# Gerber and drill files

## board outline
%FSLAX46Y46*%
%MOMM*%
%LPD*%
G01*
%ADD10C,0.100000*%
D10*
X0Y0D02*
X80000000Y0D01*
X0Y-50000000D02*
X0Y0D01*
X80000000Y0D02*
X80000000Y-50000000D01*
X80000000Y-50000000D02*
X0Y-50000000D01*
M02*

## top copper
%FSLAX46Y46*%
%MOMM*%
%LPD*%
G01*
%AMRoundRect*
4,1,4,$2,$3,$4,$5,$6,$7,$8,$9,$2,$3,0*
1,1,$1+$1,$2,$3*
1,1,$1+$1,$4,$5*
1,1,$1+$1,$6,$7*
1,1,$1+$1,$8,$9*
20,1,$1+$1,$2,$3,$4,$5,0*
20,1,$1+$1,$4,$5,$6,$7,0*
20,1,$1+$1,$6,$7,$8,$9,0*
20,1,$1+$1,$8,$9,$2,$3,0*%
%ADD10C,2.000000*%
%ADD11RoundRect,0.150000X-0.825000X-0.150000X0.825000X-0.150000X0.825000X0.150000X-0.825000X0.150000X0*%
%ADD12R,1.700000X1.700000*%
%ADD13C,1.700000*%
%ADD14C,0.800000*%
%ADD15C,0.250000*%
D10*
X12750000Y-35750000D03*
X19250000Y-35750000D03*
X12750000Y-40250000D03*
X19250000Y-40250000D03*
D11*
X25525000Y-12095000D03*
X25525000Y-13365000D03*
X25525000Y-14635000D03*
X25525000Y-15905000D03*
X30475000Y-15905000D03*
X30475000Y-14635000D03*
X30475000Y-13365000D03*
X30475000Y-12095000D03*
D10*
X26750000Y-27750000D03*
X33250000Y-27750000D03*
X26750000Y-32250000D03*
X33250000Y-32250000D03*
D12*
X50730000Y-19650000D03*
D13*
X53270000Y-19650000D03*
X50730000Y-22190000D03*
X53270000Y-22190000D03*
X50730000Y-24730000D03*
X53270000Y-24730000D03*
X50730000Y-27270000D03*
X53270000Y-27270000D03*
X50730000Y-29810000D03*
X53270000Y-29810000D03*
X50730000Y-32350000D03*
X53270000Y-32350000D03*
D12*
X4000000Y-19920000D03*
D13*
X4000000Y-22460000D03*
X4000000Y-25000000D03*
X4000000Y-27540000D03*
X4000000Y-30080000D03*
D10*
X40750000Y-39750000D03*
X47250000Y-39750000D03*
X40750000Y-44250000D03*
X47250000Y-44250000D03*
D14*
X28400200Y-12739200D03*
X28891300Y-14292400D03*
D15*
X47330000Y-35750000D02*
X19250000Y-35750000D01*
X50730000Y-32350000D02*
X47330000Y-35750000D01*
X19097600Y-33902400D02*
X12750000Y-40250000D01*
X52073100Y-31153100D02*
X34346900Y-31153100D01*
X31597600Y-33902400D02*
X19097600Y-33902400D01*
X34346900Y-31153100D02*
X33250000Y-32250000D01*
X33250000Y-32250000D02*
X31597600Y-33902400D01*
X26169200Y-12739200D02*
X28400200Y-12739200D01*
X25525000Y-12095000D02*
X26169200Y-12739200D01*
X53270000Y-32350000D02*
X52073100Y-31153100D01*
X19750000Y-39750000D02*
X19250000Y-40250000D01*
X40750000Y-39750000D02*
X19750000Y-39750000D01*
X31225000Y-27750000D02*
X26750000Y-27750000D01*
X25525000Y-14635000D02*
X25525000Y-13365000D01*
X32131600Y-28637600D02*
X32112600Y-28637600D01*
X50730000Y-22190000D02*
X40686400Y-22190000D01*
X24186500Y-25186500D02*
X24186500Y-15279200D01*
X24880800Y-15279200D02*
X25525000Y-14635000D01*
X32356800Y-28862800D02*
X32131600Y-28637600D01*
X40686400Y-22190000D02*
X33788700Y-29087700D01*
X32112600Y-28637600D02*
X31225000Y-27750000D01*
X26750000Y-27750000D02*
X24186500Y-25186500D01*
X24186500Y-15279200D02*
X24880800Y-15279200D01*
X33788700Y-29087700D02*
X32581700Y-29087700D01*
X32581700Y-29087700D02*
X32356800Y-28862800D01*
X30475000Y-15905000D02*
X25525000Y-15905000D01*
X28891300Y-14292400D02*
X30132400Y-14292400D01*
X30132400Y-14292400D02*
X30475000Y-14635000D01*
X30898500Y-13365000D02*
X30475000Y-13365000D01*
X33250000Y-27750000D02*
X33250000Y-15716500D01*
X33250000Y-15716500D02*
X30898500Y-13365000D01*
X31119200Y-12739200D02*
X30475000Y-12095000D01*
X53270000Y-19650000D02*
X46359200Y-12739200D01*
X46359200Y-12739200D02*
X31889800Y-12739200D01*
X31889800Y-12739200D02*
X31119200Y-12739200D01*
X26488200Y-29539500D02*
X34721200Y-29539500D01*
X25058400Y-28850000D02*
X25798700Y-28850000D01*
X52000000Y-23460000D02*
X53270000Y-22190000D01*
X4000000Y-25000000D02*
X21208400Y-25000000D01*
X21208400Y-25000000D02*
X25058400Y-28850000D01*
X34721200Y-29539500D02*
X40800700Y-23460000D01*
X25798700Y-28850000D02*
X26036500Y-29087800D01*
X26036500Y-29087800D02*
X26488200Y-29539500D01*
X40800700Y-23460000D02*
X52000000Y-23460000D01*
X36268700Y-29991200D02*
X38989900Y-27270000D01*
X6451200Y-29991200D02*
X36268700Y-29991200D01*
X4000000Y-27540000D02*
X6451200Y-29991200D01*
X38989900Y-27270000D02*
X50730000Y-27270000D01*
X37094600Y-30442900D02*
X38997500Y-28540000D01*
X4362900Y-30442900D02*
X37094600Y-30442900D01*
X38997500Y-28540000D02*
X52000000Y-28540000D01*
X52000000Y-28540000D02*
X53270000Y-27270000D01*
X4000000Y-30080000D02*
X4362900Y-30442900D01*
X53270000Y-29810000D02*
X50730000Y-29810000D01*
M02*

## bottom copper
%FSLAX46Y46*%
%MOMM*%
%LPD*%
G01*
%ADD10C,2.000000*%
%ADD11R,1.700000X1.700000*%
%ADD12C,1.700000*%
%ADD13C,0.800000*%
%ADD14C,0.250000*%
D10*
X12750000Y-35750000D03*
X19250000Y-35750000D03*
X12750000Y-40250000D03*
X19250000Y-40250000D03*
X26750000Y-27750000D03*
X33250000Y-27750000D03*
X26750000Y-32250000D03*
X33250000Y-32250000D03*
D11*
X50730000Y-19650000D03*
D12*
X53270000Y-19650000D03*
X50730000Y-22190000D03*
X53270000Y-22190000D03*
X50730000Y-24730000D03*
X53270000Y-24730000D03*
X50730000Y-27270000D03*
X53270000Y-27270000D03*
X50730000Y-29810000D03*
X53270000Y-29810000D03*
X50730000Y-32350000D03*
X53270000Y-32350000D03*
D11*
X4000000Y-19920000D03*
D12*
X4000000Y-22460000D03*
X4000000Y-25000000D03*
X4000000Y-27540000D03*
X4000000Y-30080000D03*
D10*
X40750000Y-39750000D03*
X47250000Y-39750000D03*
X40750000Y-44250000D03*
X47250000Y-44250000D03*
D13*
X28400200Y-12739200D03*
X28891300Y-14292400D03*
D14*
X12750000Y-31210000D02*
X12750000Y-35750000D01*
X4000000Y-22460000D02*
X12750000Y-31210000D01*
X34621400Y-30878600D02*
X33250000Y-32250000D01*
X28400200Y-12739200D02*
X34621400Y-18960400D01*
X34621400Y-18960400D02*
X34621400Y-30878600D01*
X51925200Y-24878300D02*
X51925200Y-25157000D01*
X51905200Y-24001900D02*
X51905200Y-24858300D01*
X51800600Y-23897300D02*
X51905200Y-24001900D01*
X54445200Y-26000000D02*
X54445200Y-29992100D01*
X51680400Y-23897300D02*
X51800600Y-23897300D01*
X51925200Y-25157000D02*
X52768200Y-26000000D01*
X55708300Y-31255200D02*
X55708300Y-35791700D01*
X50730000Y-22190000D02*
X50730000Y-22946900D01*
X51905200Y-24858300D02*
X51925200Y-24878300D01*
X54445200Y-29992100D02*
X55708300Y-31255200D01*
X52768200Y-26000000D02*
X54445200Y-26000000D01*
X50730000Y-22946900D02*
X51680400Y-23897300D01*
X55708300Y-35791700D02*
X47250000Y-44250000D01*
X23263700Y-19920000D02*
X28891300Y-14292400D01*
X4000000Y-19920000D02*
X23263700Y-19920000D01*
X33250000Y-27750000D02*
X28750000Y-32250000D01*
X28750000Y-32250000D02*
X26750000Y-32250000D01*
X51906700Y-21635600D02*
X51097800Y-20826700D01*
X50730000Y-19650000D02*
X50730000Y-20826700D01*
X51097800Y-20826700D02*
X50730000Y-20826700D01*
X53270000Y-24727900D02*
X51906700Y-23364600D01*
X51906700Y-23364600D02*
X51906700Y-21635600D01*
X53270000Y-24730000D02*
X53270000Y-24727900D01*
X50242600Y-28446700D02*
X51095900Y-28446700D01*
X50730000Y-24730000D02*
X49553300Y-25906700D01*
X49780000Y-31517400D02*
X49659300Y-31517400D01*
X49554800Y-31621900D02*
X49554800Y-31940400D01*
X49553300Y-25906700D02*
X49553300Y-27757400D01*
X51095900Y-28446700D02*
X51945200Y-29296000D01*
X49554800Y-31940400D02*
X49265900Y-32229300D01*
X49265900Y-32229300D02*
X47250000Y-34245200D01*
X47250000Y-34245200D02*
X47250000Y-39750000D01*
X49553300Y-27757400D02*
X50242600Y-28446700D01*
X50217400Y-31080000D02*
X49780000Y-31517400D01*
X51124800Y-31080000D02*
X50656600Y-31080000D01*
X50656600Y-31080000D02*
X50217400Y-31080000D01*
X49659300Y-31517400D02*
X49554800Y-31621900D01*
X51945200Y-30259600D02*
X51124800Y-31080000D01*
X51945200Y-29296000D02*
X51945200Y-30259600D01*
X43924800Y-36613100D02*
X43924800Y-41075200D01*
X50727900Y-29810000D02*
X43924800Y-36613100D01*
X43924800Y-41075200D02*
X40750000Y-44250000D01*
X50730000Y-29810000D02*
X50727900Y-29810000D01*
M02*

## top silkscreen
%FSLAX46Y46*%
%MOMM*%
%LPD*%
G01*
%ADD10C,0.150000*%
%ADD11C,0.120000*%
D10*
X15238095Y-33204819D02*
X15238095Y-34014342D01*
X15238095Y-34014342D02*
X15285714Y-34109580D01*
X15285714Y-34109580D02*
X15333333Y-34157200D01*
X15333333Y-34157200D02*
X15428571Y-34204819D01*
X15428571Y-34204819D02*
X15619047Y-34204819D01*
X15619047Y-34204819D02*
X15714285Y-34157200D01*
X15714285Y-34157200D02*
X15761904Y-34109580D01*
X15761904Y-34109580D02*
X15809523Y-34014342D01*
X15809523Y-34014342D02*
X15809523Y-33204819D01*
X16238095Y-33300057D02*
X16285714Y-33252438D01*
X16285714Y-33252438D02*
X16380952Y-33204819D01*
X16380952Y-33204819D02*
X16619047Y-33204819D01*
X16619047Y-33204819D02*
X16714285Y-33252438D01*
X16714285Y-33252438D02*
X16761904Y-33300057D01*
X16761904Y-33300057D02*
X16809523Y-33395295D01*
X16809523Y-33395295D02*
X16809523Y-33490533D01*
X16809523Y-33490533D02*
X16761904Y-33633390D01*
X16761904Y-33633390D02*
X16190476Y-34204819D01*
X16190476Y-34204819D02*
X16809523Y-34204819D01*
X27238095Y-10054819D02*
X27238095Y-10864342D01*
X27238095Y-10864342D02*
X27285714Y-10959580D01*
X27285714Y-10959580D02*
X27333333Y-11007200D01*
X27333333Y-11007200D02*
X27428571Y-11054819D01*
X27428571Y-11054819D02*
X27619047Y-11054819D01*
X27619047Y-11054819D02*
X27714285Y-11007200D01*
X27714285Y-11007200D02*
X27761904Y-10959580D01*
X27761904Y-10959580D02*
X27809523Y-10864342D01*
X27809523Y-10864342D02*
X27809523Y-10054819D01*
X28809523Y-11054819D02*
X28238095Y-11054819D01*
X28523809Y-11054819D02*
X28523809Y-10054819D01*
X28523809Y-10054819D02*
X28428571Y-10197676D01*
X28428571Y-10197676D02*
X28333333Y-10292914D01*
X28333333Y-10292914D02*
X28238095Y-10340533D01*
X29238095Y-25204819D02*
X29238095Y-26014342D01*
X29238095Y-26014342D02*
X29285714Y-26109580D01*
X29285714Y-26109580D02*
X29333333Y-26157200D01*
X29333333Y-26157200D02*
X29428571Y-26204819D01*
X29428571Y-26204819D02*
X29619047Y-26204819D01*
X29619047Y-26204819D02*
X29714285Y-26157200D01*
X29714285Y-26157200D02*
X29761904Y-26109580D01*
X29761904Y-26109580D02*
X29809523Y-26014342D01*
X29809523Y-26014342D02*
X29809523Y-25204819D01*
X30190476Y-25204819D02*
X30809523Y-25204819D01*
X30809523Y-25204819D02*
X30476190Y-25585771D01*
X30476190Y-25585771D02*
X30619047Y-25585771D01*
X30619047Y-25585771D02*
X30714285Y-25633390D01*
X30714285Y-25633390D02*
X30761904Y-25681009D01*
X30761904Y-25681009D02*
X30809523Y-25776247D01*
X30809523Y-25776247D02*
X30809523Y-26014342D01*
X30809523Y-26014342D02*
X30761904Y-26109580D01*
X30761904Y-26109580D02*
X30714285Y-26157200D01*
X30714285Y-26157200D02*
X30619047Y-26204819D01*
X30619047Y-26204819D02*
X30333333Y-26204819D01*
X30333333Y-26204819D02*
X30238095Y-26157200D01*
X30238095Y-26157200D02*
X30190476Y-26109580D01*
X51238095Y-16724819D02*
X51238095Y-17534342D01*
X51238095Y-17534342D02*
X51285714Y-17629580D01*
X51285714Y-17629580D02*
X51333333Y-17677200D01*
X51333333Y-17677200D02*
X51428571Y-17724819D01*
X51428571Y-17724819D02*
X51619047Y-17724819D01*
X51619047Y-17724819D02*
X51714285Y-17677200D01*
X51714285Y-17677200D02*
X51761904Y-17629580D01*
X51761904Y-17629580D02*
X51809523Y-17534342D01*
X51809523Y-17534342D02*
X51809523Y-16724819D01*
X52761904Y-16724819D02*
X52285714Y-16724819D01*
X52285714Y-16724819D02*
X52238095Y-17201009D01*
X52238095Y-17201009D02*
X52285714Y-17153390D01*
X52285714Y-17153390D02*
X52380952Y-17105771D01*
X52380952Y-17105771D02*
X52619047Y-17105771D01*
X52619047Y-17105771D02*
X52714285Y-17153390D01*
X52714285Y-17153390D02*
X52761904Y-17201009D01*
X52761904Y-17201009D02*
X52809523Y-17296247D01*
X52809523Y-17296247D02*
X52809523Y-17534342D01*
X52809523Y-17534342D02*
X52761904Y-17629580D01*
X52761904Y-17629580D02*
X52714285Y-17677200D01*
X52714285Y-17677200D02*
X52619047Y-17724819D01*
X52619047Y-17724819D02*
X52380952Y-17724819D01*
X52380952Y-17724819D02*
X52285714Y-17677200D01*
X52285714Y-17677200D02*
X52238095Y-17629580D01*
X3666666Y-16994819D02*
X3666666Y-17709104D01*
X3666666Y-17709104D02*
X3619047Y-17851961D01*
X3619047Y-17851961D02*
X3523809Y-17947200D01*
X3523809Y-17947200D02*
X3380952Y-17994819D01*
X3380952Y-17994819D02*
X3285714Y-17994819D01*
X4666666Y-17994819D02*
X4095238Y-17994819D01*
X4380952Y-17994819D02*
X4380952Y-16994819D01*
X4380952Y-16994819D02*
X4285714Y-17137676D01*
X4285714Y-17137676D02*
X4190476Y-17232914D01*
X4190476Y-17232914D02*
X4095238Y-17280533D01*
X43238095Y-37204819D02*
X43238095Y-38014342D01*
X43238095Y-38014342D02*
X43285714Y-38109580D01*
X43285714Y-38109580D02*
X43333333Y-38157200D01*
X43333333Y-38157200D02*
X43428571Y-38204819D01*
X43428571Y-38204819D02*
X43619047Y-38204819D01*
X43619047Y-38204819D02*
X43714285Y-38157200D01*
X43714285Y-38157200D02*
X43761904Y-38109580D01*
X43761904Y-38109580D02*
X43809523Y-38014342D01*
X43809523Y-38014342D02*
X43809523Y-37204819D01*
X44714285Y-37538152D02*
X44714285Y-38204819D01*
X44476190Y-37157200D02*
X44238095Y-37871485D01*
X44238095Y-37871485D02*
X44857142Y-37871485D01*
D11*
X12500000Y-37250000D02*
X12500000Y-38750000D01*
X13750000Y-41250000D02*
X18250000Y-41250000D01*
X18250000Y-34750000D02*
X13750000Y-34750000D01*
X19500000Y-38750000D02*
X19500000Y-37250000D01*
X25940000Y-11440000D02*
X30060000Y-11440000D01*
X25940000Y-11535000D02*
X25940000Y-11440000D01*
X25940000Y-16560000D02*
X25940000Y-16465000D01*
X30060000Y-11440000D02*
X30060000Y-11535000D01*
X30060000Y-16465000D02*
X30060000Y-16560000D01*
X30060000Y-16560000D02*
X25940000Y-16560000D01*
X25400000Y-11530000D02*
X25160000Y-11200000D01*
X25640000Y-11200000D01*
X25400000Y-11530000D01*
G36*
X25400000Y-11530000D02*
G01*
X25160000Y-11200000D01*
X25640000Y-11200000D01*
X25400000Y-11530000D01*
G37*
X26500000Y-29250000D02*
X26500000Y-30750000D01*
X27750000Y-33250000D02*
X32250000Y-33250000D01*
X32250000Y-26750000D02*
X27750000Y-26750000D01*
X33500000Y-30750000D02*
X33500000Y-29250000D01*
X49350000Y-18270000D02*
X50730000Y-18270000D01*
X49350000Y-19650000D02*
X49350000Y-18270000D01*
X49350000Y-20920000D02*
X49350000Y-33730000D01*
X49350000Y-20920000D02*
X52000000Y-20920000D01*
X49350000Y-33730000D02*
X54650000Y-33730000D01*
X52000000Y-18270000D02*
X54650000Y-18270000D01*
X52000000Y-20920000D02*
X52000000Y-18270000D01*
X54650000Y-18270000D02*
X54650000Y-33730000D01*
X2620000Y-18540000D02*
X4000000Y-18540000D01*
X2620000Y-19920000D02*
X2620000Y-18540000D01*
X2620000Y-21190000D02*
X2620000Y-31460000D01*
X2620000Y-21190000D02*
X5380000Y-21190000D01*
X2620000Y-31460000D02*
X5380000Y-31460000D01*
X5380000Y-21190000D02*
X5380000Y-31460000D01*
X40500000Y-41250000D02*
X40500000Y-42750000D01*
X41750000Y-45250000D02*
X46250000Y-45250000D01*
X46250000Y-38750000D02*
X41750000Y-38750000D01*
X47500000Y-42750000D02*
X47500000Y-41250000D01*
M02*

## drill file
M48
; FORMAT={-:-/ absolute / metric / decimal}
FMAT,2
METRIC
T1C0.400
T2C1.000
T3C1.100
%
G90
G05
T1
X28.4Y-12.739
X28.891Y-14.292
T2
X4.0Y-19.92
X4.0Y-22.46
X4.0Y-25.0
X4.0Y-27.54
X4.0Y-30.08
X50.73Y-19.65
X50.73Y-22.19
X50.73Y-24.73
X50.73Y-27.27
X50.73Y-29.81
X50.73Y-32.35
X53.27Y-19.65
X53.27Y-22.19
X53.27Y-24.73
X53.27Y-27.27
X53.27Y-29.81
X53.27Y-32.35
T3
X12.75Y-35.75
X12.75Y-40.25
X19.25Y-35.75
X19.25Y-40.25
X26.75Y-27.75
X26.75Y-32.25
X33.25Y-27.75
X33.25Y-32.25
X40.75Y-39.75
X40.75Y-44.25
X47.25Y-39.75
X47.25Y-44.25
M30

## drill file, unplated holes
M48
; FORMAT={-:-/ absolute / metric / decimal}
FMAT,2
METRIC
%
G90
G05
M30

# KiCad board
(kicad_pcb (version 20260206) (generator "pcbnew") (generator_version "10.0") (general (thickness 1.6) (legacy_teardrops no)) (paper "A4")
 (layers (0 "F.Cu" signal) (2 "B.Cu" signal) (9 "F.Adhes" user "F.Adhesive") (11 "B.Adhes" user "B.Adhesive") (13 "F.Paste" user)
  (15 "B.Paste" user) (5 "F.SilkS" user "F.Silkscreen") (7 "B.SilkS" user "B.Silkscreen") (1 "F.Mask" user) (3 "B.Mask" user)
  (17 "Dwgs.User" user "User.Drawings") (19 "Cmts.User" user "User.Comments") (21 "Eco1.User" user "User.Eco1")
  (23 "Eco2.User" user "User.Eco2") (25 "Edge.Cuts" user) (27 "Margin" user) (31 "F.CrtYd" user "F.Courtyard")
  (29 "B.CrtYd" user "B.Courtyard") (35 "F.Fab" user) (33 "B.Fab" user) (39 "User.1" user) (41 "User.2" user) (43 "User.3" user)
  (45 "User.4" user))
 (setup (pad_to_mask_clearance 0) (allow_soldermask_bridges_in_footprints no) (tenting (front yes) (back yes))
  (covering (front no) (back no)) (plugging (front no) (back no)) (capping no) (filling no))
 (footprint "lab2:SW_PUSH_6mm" (layer "F.Cu") (at 12.75 35.75)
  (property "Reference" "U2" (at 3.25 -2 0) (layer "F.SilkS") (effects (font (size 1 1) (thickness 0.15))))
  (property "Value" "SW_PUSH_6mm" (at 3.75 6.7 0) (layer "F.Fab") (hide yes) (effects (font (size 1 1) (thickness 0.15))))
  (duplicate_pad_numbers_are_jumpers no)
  (fp_line (start -0.25 1.5) (end -0.25 3) (stroke (width 0.12) (type solid)) (layer "F.SilkS"))
  (fp_line (start 1 5.5) (end 5.5 5.5) (stroke (width 0.12) (type solid)) (layer "F.SilkS"))
  (fp_line (start 5.5 -1) (end 1 -1) (stroke (width 0.12) (type solid)) (layer "F.SilkS"))
  (fp_line (start 6.75 3) (end 6.75 1.5) (stroke (width 0.12) (type solid)) (layer "F.SilkS"))
  (pad "1" thru_hole circle (at 0 0 90) (size 2 2) (drill 1.1) (layers "*.Cu" "*.Mask") (remove_unused_layers no) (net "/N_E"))
  (pad "2" thru_hole circle (at 6.5 0 90) (size 2 2) (drill 1.1) (layers "*.Cu" "*.Mask") (remove_unused_layers no) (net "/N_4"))
  (pad "3" thru_hole circle (at 0 4.5 90) (size 2 2) (drill 1.1) (layers "*.Cu" "*.Mask") (remove_unused_layers no) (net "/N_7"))
  (pad "4" thru_hole circle (at 6.5 4.5 90) (size 2 2) (drill 1.1) (layers "*.Cu" "*.Mask") (remove_unused_layers no) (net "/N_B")))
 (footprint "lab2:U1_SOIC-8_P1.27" (layer "F.Cu") (at 28 14)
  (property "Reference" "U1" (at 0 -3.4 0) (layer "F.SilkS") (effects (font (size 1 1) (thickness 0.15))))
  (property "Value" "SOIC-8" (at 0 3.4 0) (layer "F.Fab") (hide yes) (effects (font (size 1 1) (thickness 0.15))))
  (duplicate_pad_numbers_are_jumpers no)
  (fp_line (start -2.06 -2.56) (end 2.06 -2.56) (stroke (width 0.12) (type solid)) (layer "F.SilkS"))
  (fp_line (start -2.06 -2.465) (end -2.06 -2.56) (stroke (width 0.12) (type solid)) (layer "F.SilkS"))
  (fp_line (start -2.06 2.56) (end -2.06 2.465) (stroke (width 0.12) (type solid)) (layer "F.SilkS"))
  (fp_line (start 2.06 -2.56) (end 2.06 -2.465) (stroke (width 0.12) (type solid)) (layer "F.SilkS"))
  (fp_line (start 2.06 2.465) (end 2.06 2.56) (stroke (width 0.12) (type solid)) (layer "F.SilkS"))
  (fp_line (start 2.06 2.56) (end -2.06 2.56) (stroke (width 0.12) (type solid)) (layer "F.SilkS"))
  (fp_poly (pts (xy -2.6 -2.47) (xy -2.84 -2.8) (xy -2.36 -2.8)) (stroke (width 0.12) (type solid)) (fill yes) (layer "F.SilkS"))
  (pad "1" smd roundrect (at -2.475 -1.905) (size 1.95 0.6) (layers "F.Cu" "F.Mask" "F.Paste") (roundrect_rratio 0.25) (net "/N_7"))
  (pad "2" smd roundrect (at -2.475 -0.635) (size 1.95 0.6) (layers "F.Cu" "F.Mask" "F.Paste") (roundrect_rratio 0.25) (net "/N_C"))
  (pad "3" smd roundrect (at -2.475 0.635) (size 1.95 0.6) (layers "F.Cu" "F.Mask" "F.Paste") (roundrect_rratio 0.25) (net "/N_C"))
  (pad "4" smd roundrect (at -2.475 1.905) (size 1.95 0.6) (layers "F.Cu" "F.Mask" "F.Paste") (roundrect_rratio 0.25) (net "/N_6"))
  (pad "5" smd roundrect (at 2.475 1.905) (size 1.95 0.6) (layers "F.Cu" "F.Mask" "F.Paste") (roundrect_rratio 0.25) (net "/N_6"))
  (pad "6" smd roundrect (at 2.475 0.635) (size 1.95 0.6) (layers "F.Cu" "F.Mask" "F.Paste") (roundrect_rratio 0.25) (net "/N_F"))
  (pad "7" smd roundrect (at 2.475 -0.635) (size 1.95 0.6) (layers "F.Cu" "F.Mask" "F.Paste") (roundrect_rratio 0.25) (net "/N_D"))
  (pad "8" smd roundrect (at 2.475 -1.905) (size 1.95 0.6) (layers "F.Cu" "F.Mask" "F.Paste") (roundrect_rratio 0.25) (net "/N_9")))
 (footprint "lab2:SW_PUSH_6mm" (layer "F.Cu") (at 26.75 27.75)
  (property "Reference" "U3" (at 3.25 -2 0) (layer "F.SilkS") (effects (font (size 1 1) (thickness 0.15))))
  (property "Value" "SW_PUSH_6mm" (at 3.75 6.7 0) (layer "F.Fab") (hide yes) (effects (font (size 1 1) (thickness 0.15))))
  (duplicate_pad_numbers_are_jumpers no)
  (fp_line (start -0.25 1.5) (end -0.25 3) (stroke (width 0.12) (type solid)) (layer "F.SilkS"))
  (fp_line (start 1 5.5) (end 5.5 5.5) (stroke (width 0.12) (type solid)) (layer "F.SilkS"))
  (fp_line (start 5.5 -1) (end 1 -1) (stroke (width 0.12) (type solid)) (layer "F.SilkS"))
  (fp_line (start 6.75 3) (end 6.75 1.5) (stroke (width 0.12) (type solid)) (layer "F.SilkS"))
  (pad "1" thru_hole circle (at 0 0 90) (size 2 2) (drill 1.1) (layers "*.Cu" "*.Mask") (remove_unused_layers no) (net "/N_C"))
  (pad "2" thru_hole circle (at 6.5 0 90) (size 2 2) (drill 1.1) (layers "*.Cu" "*.Mask") (remove_unused_layers no) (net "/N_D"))
  (pad "3" thru_hole circle (at 0 4.5 90) (size 2 2) (drill 1.1) (layers "*.Cu" "*.Mask") (remove_unused_layers no) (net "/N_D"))
  (pad "4" thru_hole circle (at 6.5 4.5 90) (size 2 2) (drill 1.1) (layers "*.Cu" "*.Mask") (remove_unused_layers no) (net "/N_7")))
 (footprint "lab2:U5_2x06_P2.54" (layer "F.Cu") (at 50.73 19.65)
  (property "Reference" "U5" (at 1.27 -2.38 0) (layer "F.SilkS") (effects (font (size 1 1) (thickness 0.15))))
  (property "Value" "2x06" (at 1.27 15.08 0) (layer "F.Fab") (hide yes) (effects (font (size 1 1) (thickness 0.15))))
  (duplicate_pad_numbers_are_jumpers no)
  (fp_line (start -1.38 -1.38) (end 0 -1.38) (stroke (width 0.12) (type solid)) (layer "F.SilkS"))
  (fp_line (start -1.38 0) (end -1.38 -1.38) (stroke (width 0.12) (type solid)) (layer "F.SilkS"))
  (fp_line (start -1.38 1.27) (end -1.38 14.08) (stroke (width 0.12) (type solid)) (layer "F.SilkS"))
  (fp_line (start -1.38 1.27) (end 1.27 1.27) (stroke (width 0.12) (type solid)) (layer "F.SilkS"))
  (fp_line (start -1.38 14.08) (end 3.92 14.08) (stroke (width 0.12) (type solid)) (layer "F.SilkS"))
  (fp_line (start 1.27 -1.38) (end 3.92 -1.38) (stroke (width 0.12) (type solid)) (layer "F.SilkS"))
  (fp_line (start 1.27 1.27) (end 1.27 -1.38) (stroke (width 0.12) (type solid)) (layer "F.SilkS"))
  (fp_line (start 3.92 -1.38) (end 3.92 14.08) (stroke (width 0.12) (type solid)) (layer "F.SilkS"))
  (pad "1" thru_hole rect (at 0 0) (size 1.7 1.7) (drill 1) (layers "*.Cu" "*.Mask") (remove_unused_layers no) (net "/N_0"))
  (pad "2" thru_hole circle (at 2.54 0) (size 1.7 1.7) (drill 1) (layers "*.Cu" "*.Mask") (remove_unused_layers no) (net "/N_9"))
  (pad "3" thru_hole circle (at 0 2.54) (size 1.7 1.7) (drill 1) (layers "*.Cu" "*.Mask") (remove_unused_layers no) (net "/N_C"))
  (pad "4" thru_hole circle (at 2.54 2.54) (size 1.7 1.7) (drill 1) (layers "*.Cu" "*.Mask") (remove_unused_layers no) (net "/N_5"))
  (pad "5" thru_hole circle (at 0 5.08) (size 1.7 1.7) (drill 1) (layers "*.Cu" "*.Mask") (remove_unused_layers no) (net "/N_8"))
  (pad "6" thru_hole circle (at 2.54 5.08) (size 1.7 1.7) (drill 1) (layers "*.Cu" "*.Mask") (remove_unused_layers no) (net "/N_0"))
  (pad "7" thru_hole circle (at 0 7.62) (size 1.7 1.7) (drill 1) (layers "*.Cu" "*.Mask") (remove_unused_layers no) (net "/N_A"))
  (pad "8" thru_hole circle (at 2.54 7.62) (size 1.7 1.7) (drill 1) (layers "*.Cu" "*.Mask") (remove_unused_layers no) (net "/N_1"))
  (pad "9" thru_hole circle (at 0 10.16) (size 1.7 1.7) (drill 1) (layers "*.Cu" "*.Mask") (remove_unused_layers no) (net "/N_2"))
  (pad "10" thru_hole circle (at 2.54 10.16) (size 1.7 1.7) (drill 1) (layers "*.Cu" "*.Mask") (remove_unused_layers no) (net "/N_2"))
  (pad "11" thru_hole circle (at 0 12.7) (size 1.7 1.7) (drill 1) (layers "*.Cu" "*.Mask") (remove_unused_layers no) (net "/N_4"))
  (pad "12" thru_hole circle (at 2.54 12.7) (size 1.7 1.7) (drill 1) (layers "*.Cu" "*.Mask") (remove_unused_layers no) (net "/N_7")))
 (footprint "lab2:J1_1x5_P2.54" (layer "F.Cu") (at 4 19.92)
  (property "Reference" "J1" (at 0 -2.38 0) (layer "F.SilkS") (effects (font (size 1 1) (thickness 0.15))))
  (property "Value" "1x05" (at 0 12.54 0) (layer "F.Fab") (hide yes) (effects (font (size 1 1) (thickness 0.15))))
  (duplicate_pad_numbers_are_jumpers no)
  (fp_line (start -1.38 -1.38) (end 0 -1.38) (stroke (width 0.12) (type solid)) (layer "F.SilkS"))
  (fp_line (start -1.38 0) (end -1.38 -1.38) (stroke (width 0.12) (type solid)) (layer "F.SilkS"))
  (fp_line (start -1.38 1.27) (end -1.38 11.54) (stroke (width 0.12) (type solid)) (layer "F.SilkS"))
  (fp_line (start -1.38 1.27) (end 1.38 1.27) (stroke (width 0.12) (type solid)) (layer "F.SilkS"))
  (fp_line (start -1.38 11.54) (end 1.38 11.54) (stroke (width 0.12) (type solid)) (layer "F.SilkS"))
  (fp_line (start 1.38 1.27) (end 1.38 11.54) (stroke (width 0.12) (type solid)) (layer "F.SilkS"))
  (pad "1" thru_hole rect (at 0 0) (size 1.7 1.7) (drill 1) (layers "*.Cu" "*.Mask") (remove_unused_layers no) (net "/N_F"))
  (pad "2" thru_hole circle (at 0 2.54) (size 1.7 1.7) (drill 1) (layers "*.Cu" "*.Mask") (remove_unused_layers no) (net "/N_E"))
  (pad "3" thru_hole circle (at 0 5.08) (size 1.7 1.7) (drill 1) (layers "*.Cu" "*.Mask") (remove_unused_layers no) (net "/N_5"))
  (pad "4" thru_hole circle (at 0 7.62) (size 1.7 1.7) (drill 1) (layers "*.Cu" "*.Mask") (remove_unused_layers no) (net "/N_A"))
  (pad "5" thru_hole circle (at 0 10.16) (size 1.7 1.7) (drill 1) (layers "*.Cu" "*.Mask") (remove_unused_layers no) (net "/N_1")))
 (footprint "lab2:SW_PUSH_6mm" (layer "F.Cu") (at 40.75 39.75)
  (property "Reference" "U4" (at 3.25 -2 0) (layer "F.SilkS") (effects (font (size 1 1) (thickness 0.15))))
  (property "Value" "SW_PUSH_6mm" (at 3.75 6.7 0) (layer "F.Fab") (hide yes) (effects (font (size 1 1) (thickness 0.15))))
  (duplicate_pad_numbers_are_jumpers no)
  (fp_line (start -0.25 1.5) (end -0.25 3) (stroke (width 0.12) (type solid)) (layer "F.SilkS"))
  (fp_line (start 1 5.5) (end 5.5 5.5) (stroke (width 0.12) (type solid)) (layer "F.SilkS"))
  (fp_line (start 5.5 -1) (end 1 -1) (stroke (width 0.12) (type solid)) (layer "F.SilkS"))
  (fp_line (start 6.75 3) (end 6.75 1.5) (stroke (width 0.12) (type solid)) (layer "F.SilkS"))
  (pad "1" thru_hole circle (at 0 0 90) (size 2 2) (drill 1.1) (layers "*.Cu" "*.Mask") (remove_unused_layers no) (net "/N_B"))
  (pad "2" thru_hole circle (at 6.5 0 90) (size 2 2) (drill 1.1) (layers "*.Cu" "*.Mask") (remove_unused_layers no) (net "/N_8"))
  (pad "3" thru_hole circle (at 0 4.5 90) (size 2 2) (drill 1.1) (layers "*.Cu" "*.Mask") (remove_unused_layers no) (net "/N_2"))
  (pad "4" thru_hole circle (at 6.5 4.5 90) (size 2 2) (drill 1.1) (layers "*.Cu" "*.Mask") (remove_unused_layers no) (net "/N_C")))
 (gr_line (start 0 0) (end 80 0) (stroke (width 0.1) (type default)) (layer "Edge.Cuts"))
 (gr_line (start 0 50) (end 0 0) (stroke (width 0.1) (type default)) (layer "Edge.Cuts"))
 (gr_line (start 80 0) (end 80 50) (stroke (width 0.1) (type default)) (layer "Edge.Cuts"))
 (gr_line (start 80 50) (end 0 50) (stroke (width 0.1) (type default)) (layer "Edge.Cuts"))
 (segment (start 12.75 31.21) (end 12.75 35.75) (width 0.25) (layer "B.Cu") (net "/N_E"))
 (segment (start 4 22.46) (end 12.75 31.21) (width 0.25) (layer "B.Cu") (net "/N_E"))
 (segment (start 47.33 35.75) (end 19.25 35.75) (width 0.25) (layer "F.Cu") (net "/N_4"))
 (segment (start 50.73 32.35) (end 47.33 35.75) (width 0.25) (layer "F.Cu") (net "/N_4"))
 (segment (start 19.0976 33.9024) (end 12.75 40.25) (width 0.25) (layer "F.Cu") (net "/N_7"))
 (segment (start 52.0731 31.1531) (end 34.3469 31.1531) (width 0.25) (layer "F.Cu") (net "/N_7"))
 (segment (start 31.5976 33.9024) (end 19.0976 33.9024) (width 0.25) (layer "F.Cu") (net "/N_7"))
 (segment (start 34.3469 31.1531) (end 33.25 32.25) (width 0.25) (layer "F.Cu") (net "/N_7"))
 (segment (start 33.25 32.25) (end 31.5976 33.9024) (width 0.25) (layer "F.Cu") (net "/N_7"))
 (segment (start 26.1692 12.7392) (end 28.4002 12.7392) (width 0.25) (layer "F.Cu") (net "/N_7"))
 (segment (start 25.525 12.095) (end 26.1692 12.7392) (width 0.25) (layer "F.Cu") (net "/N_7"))
 (segment (start 53.27 32.35) (end 52.0731 31.1531) (width 0.25) (layer "F.Cu") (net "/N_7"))
 (via (at 28.4002 12.7392) (size 0.8) (drill 0.4) (layers "F.Cu" "B.Cu") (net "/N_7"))
 (segment (start 34.6214 30.8786) (end 33.25 32.25) (width 0.25) (layer "B.Cu") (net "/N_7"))
 (segment (start 28.4002 12.7392) (end 34.6214 18.9604) (width 0.25) (layer "B.Cu") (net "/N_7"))
 (segment (start 34.6214 18.9604) (end 34.6214 30.8786) (width 0.25) (layer "B.Cu") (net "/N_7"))
 (segment (start 19.75 39.75) (end 19.25 40.25) (width 0.25) (layer "F.Cu") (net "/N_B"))
 (segment (start 40.75 39.75) (end 19.75 39.75) (width 0.25) (layer "F.Cu") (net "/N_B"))
 (segment (start 31.225 27.75) (end 26.75 27.75) (width 0.25) (layer "F.Cu") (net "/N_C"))
 (segment (start 25.525 14.635) (end 25.525 13.365) (width 0.25) (layer "F.Cu") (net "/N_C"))
 (segment (start 32.1316 28.6376) (end 32.1126 28.6376) (width 0.25) (layer "F.Cu") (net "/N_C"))
 (segment (start 50.73 22.19) (end 40.6864 22.19) (width 0.25) (layer "F.Cu") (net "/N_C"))
 (segment (start 24.1865 25.1865) (end 24.1865 15.2792) (width 0.25) (layer "F.Cu") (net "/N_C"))
 (segment (start 24.8808 15.2792) (end 25.525 14.635) (width 0.25) (layer "F.Cu") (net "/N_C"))
 (segment (start 32.3568 28.8628) (end 32.1316 28.6376) (width 0.25) (layer "F.Cu") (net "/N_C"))
 (segment (start 40.6864 22.19) (end 33.7887 29.0877) (width 0.25) (layer "F.Cu") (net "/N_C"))
 (segment (start 32.1126 28.6376) (end 31.225 27.75) (width 0.25) (layer "F.Cu") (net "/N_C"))
 (segment (start 26.75 27.75) (end 24.1865 25.1865) (width 0.25) (layer "F.Cu") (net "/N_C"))
 (segment (start 24.1865 15.2792) (end 24.8808 15.2792) (width 0.25) (layer "F.Cu") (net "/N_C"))
 (segment (start 33.7887 29.0877) (end 32.5817 29.0877) (width 0.25) (layer "F.Cu") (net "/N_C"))
 (segment (start 32.5817 29.0877) (end 32.3568 28.8628) (width 0.25) (layer "F.Cu") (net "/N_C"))
 (segment (start 51.9252 24.8783) (end 51.9252 25.157) (width 0.25) (layer "B.Cu") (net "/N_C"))
 (segment (start 51.9052 24.0019) (end 51.9052 24.8583) (width 0.25) (layer "B.Cu") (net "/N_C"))
 (segment (start 51.8006 23.8973) (end 51.9052 24.0019) (width 0.25) (layer "B.Cu") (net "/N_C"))
 (segment (start 54.4452 26) (end 54.4452 29.9921) (width 0.25) (layer "B.Cu") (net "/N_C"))
 (segment (start 51.6804 23.8973) (end 51.8006 23.8973) (width 0.25) (layer "B.Cu") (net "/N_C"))
 (segment (start 51.9252 25.157) (end 52.7682 26) (width 0.25) (layer "B.Cu") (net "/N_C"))
 (segment (start 55.7083 31.2552) (end 55.7083 35.7917) (width 0.25) (layer "B.Cu") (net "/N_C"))
 (segment (start 50.73 22.19) (end 50.73 22.9469) (width 0.25) (layer "B.Cu") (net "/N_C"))
 (segment (start 51.9052 24.8583) (end 51.9252 24.8783) (width 0.25) (layer "B.Cu") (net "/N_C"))
 (segment (start 54.4452 29.9921) (end 55.7083 31.2552) (width 0.25) (layer "B.Cu") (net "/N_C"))
 (segment (start 52.7682 26) (end 54.4452 26) (width 0.25) (layer "B.Cu") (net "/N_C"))
 (segment (start 50.73 22.9469) (end 51.6804 23.8973) (width 0.25) (layer "B.Cu") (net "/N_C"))
 (segment (start 55.7083 35.7917) (end 47.25 44.25) (width 0.25) (layer "B.Cu") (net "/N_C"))
 (segment (start 30.475 15.905) (end 25.525 15.905) (width 0.25) (layer "F.Cu") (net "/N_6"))
 (segment (start 28.8913 14.2924) (end 30.1324 14.2924) (width 0.25) (layer "F.Cu") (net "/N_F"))
 (segment (start 30.1324 14.2924) (end 30.475 14.635) (width 0.25) (layer "F.Cu") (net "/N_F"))
 (via (at 28.8913 14.2924) (size 0.8) (drill 0.4) (layers "F.Cu" "B.Cu") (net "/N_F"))
 (segment (start 23.2637 19.92) (end 28.8913 14.2924) (width 0.25) (layer "B.Cu") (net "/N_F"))
 (segment (start 4 19.92) (end 23.2637 19.92) (width 0.25) (layer "B.Cu") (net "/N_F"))
 (segment (start 30.8985 13.365) (end 30.475 13.365) (width 0.25) (layer "F.Cu") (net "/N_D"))
 (segment (start 33.25 27.75) (end 33.25 15.7165) (width 0.25) (layer "F.Cu") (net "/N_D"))
 (segment (start 33.25 15.7165) (end 30.8985 13.365) (width 0.25) (layer "F.Cu") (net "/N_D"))
 (segment (start 33.25 27.75) (end 28.75 32.25) (width 0.25) (layer "B.Cu") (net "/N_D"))
 (segment (start 28.75 32.25) (end 26.75 32.25) (width 0.25) (layer "B.Cu") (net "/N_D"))
 (segment (start 31.1192 12.7392) (end 30.475 12.095) (width 0.25) (layer "F.Cu") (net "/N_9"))
 (segment (start 53.27 19.65) (end 46.3592 12.7392) (width 0.25) (layer "F.Cu") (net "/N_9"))
 (segment (start 46.3592 12.7392) (end 31.8898 12.7392) (width 0.25) (layer "F.Cu") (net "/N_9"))
 (segment (start 31.8898 12.7392) (end 31.1192 12.7392) (width 0.25) (layer "F.Cu") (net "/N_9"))
 (segment (start 51.9067 21.6356) (end 51.0978 20.8267) (width 0.25) (layer "B.Cu") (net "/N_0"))
 (segment (start 50.73 19.65) (end 50.73 20.8267) (width 0.25) (layer "B.Cu") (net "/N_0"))
 (segment (start 51.0978 20.8267) (end 50.73 20.8267) (width 0.25) (layer "B.Cu") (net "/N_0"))
 (segment (start 53.27 24.7279) (end 51.9067 23.3646) (width 0.25) (layer "B.Cu") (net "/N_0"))
 (segment (start 51.9067 23.3646) (end 51.9067 21.6356) (width 0.25) (layer "B.Cu") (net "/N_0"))
 (segment (start 53.27 24.73) (end 53.27 24.7279) (width 0.25) (layer "B.Cu") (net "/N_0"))
 (segment (start 26.4882 29.5395) (end 34.7212 29.5395) (width 0.25) (layer "F.Cu") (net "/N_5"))
 (segment (start 25.0584 28.85) (end 25.7987 28.85) (width 0.25) (layer "F.Cu") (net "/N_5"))
 (segment (start 52 23.46) (end 53.27 22.19) (width 0.25) (layer "F.Cu") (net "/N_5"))
 (segment (start 4 25) (end 21.2084 25) (width 0.25) (layer "F.Cu") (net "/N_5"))
 (segment (start 21.2084 25) (end 25.0584 28.85) (width 0.25) (layer "F.Cu") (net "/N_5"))
 (segment (start 34.7212 29.5395) (end 40.8007 23.46) (width 0.25) (layer "F.Cu") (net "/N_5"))
 (segment (start 25.7987 28.85) (end 26.0365 29.0878) (width 0.25) (layer "F.Cu") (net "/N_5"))
 (segment (start 26.0365 29.0878) (end 26.4882 29.5395) (width 0.25) (layer "F.Cu") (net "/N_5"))
 (segment (start 40.8007 23.46) (end 52 23.46) (width 0.25) (layer "F.Cu") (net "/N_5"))
 (segment (start 50.2426 28.4467) (end 51.0959 28.4467) (width 0.25) (layer "B.Cu") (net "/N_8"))
 (segment (start 50.73 24.73) (end 49.5533 25.9067) (width 0.25) (layer "B.Cu") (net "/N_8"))
 (segment (start 49.78 31.5174) (end 49.6593 31.5174) (width 0.25) (layer "B.Cu") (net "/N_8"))
 (segment (start 49.5548 31.6219) (end 49.5548 31.9404) (width 0.25) (layer "B.Cu") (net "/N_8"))
 (segment (start 49.5533 25.9067) (end 49.5533 27.7574) (width 0.25) (layer "B.Cu") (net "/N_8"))
 (segment (start 51.0959 28.4467) (end 51.9452 29.296) (width 0.25) (layer "B.Cu") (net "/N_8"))
 (segment (start 49.5548 31.9404) (end 49.2659 32.2293) (width 0.25) (layer "B.Cu") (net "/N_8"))
 (segment (start 49.2659 32.2293) (end 47.25 34.2452) (width 0.25) (layer "B.Cu") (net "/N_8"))
 (segment (start 47.25 34.2452) (end 47.25 39.75) (width 0.25) (layer "B.Cu") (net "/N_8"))
 (segment (start 49.5533 27.7574) (end 50.2426 28.4467) (width 0.25) (layer "B.Cu") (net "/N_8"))
 (segment (start 50.2174 31.08) (end 49.78 31.5174) (width 0.25) (layer "B.Cu") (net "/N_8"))
 (segment (start 51.1248 31.08) (end 50.6566 31.08) (width 0.25) (layer "B.Cu") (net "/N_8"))
 (segment (start 50.6566 31.08) (end 50.2174 31.08) (width 0.25) (layer "B.Cu") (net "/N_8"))
 (segment (start 49.6593 31.5174) (end 49.5548 31.6219) (width 0.25) (layer "B.Cu") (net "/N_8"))
 (segment (start 51.9452 30.2596) (end 51.1248 31.08) (width 0.25) (layer "B.Cu") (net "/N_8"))
 (segment (start 51.9452 29.296) (end 51.9452 30.2596) (width 0.25) (layer "B.Cu") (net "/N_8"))
 (segment (start 36.2687 29.9912) (end 38.9899 27.27) (width 0.25) (layer "F.Cu") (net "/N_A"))
 (segment (start 6.4512 29.9912) (end 36.2687 29.9912) (width 0.25) (layer "F.Cu") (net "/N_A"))
 (segment (start 4 27.54) (end 6.4512 29.9912) (width 0.25) (layer "F.Cu") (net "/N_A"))
 (segment (start 38.9899 27.27) (end 50.73 27.27) (width 0.25) (layer "F.Cu") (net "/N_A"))
 (segment (start 37.0946 30.4429) (end 38.9975 28.54) (width 0.25) (layer "F.Cu") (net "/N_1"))
 (segment (start 4.3629 30.4429) (end 37.0946 30.4429) (width 0.25) (layer "F.Cu") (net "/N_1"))
 (segment (start 38.9975 28.54) (end 52 28.54) (width 0.25) (layer "F.Cu") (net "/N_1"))
 (segment (start 52 28.54) (end 53.27 27.27) (width 0.25) (layer "F.Cu") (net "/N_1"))
 (segment (start 4 30.08) (end 4.3629 30.4429) (width 0.25) (layer "F.Cu") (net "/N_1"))
 (segment (start 53.27 29.81) (end 50.73 29.81) (width 0.25) (layer "F.Cu") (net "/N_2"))
 (segment (start 43.9248 36.6131) (end 43.9248 41.0752) (width 0.25) (layer "B.Cu") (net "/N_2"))
 (segment (start 50.7279 29.81) (end 43.9248 36.6131) (width 0.25) (layer "B.Cu") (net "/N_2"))
 (segment (start 43.9248 41.0752) (end 40.75 44.25) (width 0.25) (layer "B.Cu") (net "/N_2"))
 (segment (start 50.73 29.81) (end 50.7279 29.81) (width 0.25) (layer "B.Cu") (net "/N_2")))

